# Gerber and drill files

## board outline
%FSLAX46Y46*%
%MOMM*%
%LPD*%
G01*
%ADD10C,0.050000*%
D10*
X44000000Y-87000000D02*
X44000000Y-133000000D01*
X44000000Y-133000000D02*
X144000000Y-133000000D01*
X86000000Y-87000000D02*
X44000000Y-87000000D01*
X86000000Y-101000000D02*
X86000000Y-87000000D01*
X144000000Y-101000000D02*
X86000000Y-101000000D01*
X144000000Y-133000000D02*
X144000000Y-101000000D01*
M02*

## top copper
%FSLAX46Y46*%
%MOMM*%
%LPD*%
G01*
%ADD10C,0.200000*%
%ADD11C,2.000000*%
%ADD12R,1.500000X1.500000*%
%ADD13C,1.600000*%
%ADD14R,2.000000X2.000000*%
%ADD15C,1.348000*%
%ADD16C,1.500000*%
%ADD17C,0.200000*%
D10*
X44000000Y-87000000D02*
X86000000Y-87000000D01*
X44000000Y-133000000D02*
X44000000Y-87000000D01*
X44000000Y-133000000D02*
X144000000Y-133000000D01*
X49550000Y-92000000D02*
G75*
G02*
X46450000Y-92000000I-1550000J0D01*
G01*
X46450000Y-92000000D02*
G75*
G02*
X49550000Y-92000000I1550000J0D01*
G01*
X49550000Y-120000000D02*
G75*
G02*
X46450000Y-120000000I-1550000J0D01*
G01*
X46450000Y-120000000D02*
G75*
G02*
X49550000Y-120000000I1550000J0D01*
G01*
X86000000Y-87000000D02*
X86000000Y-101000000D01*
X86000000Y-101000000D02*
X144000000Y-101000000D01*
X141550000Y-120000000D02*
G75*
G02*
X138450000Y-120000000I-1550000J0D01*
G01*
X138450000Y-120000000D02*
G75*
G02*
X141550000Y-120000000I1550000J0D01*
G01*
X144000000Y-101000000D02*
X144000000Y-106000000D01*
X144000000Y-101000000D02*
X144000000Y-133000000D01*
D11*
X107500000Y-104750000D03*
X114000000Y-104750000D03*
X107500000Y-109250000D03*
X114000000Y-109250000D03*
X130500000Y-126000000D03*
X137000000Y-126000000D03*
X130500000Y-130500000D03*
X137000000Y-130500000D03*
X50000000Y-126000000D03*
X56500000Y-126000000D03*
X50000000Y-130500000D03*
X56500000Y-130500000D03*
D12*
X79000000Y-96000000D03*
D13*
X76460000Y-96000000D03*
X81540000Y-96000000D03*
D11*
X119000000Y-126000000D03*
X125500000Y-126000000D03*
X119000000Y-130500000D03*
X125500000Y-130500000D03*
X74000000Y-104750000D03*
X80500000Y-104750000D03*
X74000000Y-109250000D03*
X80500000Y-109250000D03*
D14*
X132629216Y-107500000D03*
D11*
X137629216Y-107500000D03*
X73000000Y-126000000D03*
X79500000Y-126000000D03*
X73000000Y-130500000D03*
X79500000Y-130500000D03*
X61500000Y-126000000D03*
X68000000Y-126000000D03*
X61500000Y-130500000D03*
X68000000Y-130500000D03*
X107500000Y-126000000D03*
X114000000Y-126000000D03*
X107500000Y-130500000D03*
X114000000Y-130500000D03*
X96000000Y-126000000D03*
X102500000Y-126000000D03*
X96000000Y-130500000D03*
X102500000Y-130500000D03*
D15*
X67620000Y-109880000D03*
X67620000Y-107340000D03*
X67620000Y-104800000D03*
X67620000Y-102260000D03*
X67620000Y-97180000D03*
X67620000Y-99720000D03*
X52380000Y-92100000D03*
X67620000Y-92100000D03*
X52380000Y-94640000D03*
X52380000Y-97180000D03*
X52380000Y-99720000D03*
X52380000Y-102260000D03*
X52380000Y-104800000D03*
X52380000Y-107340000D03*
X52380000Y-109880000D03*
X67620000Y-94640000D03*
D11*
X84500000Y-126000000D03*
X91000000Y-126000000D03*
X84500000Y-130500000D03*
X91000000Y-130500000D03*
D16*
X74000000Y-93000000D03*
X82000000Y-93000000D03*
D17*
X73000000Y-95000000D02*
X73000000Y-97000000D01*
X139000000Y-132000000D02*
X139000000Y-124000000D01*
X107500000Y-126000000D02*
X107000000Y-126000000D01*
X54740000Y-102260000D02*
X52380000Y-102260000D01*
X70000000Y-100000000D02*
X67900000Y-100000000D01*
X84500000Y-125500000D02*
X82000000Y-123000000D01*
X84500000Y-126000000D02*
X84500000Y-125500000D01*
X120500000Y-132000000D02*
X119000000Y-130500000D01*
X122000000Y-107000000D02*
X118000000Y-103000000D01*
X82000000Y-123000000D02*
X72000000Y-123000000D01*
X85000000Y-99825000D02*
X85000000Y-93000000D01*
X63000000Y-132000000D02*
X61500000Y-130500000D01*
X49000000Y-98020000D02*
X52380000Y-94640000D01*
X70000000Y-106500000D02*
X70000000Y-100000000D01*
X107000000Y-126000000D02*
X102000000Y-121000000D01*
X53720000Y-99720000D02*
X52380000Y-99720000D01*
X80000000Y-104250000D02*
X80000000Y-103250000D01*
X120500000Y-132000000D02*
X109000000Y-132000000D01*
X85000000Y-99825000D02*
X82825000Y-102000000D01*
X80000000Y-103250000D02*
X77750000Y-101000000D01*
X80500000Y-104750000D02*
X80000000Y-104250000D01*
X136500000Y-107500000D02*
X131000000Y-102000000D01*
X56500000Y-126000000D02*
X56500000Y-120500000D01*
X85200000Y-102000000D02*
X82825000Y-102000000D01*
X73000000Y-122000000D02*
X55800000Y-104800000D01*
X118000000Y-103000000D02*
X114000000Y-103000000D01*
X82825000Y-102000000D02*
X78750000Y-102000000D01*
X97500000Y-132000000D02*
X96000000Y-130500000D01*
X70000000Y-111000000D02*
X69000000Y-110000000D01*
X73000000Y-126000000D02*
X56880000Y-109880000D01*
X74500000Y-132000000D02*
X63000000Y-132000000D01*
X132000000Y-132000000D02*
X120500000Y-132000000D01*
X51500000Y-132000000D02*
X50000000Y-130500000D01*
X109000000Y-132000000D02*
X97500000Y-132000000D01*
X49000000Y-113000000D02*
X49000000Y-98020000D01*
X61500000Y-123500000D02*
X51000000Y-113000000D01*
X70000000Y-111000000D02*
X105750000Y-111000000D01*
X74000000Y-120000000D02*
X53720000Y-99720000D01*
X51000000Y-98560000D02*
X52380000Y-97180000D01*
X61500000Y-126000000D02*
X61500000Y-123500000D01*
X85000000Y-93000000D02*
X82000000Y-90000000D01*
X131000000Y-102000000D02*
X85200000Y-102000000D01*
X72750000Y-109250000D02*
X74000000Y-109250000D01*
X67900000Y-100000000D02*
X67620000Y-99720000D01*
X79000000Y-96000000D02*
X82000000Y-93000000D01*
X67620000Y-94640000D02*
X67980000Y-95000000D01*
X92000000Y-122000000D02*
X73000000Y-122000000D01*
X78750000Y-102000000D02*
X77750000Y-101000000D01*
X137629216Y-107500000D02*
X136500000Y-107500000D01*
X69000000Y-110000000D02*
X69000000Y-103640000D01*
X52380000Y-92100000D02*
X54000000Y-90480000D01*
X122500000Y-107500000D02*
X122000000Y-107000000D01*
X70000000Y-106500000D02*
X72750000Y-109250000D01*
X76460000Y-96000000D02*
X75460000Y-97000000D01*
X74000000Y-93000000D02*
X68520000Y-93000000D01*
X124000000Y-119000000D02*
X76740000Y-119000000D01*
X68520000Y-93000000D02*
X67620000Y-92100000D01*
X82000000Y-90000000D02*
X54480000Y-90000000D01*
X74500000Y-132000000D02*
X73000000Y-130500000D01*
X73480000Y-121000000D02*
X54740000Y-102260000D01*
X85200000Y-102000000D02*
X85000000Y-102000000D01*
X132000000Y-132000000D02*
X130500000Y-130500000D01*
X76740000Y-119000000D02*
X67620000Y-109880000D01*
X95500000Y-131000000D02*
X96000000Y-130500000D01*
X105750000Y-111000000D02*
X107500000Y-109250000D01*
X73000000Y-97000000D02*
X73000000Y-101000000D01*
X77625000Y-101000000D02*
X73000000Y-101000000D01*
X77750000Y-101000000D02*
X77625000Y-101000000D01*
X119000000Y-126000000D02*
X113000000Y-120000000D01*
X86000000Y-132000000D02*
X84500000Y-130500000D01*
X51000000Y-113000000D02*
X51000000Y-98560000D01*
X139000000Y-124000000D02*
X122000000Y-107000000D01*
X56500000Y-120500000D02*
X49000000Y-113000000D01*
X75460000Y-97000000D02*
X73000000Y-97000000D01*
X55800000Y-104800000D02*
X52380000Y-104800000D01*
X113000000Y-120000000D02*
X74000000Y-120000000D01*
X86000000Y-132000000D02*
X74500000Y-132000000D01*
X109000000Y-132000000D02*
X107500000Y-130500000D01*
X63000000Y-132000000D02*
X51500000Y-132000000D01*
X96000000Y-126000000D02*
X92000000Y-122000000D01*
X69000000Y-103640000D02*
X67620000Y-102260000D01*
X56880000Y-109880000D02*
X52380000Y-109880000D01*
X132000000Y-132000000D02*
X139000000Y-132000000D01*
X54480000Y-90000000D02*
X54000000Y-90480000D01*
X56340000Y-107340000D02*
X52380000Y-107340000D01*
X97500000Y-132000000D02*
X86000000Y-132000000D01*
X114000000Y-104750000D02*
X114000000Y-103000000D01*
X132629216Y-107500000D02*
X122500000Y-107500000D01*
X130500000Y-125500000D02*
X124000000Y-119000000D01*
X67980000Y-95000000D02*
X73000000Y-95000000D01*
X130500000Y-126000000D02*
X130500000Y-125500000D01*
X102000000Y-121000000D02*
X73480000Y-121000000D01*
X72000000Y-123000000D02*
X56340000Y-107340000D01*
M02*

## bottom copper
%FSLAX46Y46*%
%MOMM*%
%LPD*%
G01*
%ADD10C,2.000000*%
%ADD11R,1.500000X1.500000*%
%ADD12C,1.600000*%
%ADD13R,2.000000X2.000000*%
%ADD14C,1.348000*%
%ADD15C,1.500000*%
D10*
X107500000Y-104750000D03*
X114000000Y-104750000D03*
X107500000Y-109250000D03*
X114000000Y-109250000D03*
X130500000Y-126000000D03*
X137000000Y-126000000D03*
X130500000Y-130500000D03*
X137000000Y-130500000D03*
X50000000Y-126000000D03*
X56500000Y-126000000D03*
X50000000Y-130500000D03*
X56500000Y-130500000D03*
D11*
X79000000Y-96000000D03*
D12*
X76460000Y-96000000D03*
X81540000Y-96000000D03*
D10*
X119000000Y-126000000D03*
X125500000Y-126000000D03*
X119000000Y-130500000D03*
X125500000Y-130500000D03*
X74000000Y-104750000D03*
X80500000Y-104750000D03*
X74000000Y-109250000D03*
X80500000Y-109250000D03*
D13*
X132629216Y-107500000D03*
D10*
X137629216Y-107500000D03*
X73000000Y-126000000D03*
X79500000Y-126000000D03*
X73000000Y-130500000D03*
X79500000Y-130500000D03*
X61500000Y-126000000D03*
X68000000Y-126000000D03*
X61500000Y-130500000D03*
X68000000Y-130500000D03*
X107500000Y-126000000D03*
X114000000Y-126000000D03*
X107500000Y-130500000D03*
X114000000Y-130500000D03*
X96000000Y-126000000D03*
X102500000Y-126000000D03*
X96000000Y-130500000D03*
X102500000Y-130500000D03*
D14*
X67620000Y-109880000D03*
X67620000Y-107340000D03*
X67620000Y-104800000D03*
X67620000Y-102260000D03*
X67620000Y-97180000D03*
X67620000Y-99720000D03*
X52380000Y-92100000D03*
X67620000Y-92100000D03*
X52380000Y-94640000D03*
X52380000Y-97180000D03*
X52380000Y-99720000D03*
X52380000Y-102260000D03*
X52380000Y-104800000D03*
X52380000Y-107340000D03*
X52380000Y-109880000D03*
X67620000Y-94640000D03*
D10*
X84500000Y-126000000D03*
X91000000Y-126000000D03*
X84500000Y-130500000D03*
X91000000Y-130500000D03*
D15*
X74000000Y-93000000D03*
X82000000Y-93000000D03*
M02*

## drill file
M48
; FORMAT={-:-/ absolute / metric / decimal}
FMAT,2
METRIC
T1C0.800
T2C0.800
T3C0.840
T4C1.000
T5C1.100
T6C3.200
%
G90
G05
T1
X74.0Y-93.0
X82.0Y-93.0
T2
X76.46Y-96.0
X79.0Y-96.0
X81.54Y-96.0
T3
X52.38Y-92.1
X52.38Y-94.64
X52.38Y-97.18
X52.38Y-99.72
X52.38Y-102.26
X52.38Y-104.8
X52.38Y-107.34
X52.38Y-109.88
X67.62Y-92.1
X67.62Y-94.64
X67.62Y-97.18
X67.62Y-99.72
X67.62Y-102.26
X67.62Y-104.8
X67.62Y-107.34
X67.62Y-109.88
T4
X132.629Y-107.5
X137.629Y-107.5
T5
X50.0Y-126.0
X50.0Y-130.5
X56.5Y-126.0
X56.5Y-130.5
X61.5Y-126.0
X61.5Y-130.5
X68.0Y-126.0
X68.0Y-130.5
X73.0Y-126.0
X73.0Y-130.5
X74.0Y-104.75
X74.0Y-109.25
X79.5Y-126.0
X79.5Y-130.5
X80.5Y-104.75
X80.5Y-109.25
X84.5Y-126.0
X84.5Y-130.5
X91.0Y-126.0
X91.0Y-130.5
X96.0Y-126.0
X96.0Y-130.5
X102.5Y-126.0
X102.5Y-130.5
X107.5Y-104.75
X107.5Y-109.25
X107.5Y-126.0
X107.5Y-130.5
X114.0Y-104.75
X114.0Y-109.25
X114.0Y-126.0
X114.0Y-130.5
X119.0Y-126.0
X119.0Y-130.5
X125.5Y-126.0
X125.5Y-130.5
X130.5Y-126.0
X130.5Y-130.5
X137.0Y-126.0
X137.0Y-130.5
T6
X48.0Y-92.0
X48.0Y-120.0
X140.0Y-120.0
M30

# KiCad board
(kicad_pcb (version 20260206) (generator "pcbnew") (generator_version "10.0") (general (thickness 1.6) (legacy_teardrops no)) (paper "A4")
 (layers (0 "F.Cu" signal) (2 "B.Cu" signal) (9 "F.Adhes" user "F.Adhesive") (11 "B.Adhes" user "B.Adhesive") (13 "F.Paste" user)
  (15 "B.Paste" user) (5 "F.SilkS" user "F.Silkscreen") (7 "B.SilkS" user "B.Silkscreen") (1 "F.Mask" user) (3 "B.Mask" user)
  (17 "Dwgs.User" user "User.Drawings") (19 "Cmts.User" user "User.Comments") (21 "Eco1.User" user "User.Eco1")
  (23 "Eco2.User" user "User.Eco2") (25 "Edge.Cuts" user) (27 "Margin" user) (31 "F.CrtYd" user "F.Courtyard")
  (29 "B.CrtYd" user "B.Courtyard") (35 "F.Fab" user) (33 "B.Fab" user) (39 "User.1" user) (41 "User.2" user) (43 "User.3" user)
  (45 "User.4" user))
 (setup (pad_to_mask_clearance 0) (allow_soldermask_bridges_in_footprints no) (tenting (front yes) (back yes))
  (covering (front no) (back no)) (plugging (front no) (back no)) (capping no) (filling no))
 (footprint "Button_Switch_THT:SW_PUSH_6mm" (layer "F.Cu") (at 107.5 104.75)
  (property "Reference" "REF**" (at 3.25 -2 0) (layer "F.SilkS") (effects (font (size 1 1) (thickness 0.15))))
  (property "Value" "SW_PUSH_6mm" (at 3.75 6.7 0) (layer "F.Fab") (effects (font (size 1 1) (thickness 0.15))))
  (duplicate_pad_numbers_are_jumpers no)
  (pad "1" thru_hole circle (at 0 0 90) (size 2 2) (drill 1.1) (layers "*.Cu" "*.Mask") (remove_unused_layers no))
  (pad "1" thru_hole circle (at 6.5 0 90) (size 2 2) (drill 1.1) (layers "*.Cu" "*.Mask") (remove_unused_layers no))
  (pad "2" thru_hole circle (at 0 4.5 90) (size 2 2) (drill 1.1) (layers "*.Cu" "*.Mask") (remove_unused_layers no))
  (pad "2" thru_hole circle (at 6.5 4.5 90) (size 2 2) (drill 1.1) (layers "*.Cu" "*.Mask") (remove_unused_layers no)))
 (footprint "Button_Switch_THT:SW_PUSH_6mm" (layer "F.Cu") (at 130.5 126)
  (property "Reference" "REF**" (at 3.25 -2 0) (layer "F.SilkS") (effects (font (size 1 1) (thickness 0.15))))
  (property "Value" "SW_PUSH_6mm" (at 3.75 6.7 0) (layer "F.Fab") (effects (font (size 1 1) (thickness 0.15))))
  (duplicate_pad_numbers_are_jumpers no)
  (pad "1" thru_hole circle (at 0 0 90) (size 2 2) (drill 1.1) (layers "*.Cu" "*.Mask") (remove_unused_layers no))
  (pad "1" thru_hole circle (at 6.5 0 90) (size 2 2) (drill 1.1) (layers "*.Cu" "*.Mask") (remove_unused_layers no))
  (pad "2" thru_hole circle (at 0 4.5 90) (size 2 2) (drill 1.1) (layers "*.Cu" "*.Mask") (remove_unused_layers no))
  (pad "2" thru_hole circle (at 6.5 4.5 90) (size 2 2) (drill 1.1) (layers "*.Cu" "*.Mask") (remove_unused_layers no)))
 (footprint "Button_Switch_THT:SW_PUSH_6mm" (layer "F.Cu") (at 50 126)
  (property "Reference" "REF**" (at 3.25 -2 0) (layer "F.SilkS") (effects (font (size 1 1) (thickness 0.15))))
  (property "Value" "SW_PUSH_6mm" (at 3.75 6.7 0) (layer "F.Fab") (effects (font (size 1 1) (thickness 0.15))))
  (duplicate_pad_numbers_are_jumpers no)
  (pad "1" thru_hole circle (at 0 0 90) (size 2 2) (drill 1.1) (layers "*.Cu" "*.Mask") (remove_unused_layers no))
  (pad "1" thru_hole circle (at 6.5 0 90) (size 2 2) (drill 1.1) (layers "*.Cu" "*.Mask") (remove_unused_layers no))
  (pad "2" thru_hole circle (at 0 4.5 90) (size 2 2) (drill 1.1) (layers "*.Cu" "*.Mask") (remove_unused_layers no))
  (pad "2" thru_hole circle (at 6.5 4.5 90) (size 2 2) (drill 1.1) (layers "*.Cu" "*.Mask") (remove_unused_layers no)))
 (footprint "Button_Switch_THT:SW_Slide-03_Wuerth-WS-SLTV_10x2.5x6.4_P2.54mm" (layer "F.Cu") (at 79 96)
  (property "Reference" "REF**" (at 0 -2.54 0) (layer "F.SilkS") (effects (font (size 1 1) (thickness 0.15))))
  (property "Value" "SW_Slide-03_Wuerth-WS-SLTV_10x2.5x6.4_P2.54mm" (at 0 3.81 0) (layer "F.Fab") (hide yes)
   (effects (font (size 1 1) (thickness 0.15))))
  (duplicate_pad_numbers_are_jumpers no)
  (pad "1" thru_hole rect (at 0 0) (size 1.5 1.5) (drill 0.8) (layers "*.Cu" "*.Mask") (remove_unused_layers no))
  (pad "2" thru_hole circle (at -2.54 0) (size 1.6 1.6) (drill 0.8) (layers "*.Cu" "*.Mask") (remove_unused_layers no))
  (pad "3" thru_hole circle (at 2.54 0) (size 1.6 1.6) (drill 0.8) (layers "*.Cu" "*.Mask") (remove_unused_layers no)))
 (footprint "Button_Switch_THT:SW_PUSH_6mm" (layer "F.Cu") (at 119 126)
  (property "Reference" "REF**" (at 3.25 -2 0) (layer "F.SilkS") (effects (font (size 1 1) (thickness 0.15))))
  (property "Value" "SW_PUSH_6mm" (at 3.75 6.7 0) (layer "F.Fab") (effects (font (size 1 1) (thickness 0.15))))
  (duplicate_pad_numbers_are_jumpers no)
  (pad "1" thru_hole circle (at 0 0 90) (size 2 2) (drill 1.1) (layers "*.Cu" "*.Mask") (remove_unused_layers no))
  (pad "1" thru_hole circle (at 6.5 0 90) (size 2 2) (drill 1.1) (layers "*.Cu" "*.Mask") (remove_unused_layers no))
  (pad "2" thru_hole circle (at 0 4.5 90) (size 2 2) (drill 1.1) (layers "*.Cu" "*.Mask") (remove_unused_layers no))
  (pad "2" thru_hole circle (at 6.5 4.5 90) (size 2 2) (drill 1.1) (layers "*.Cu" "*.Mask") (remove_unused_layers no)))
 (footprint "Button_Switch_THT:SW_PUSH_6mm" (layer "F.Cu") (at 74 104.75)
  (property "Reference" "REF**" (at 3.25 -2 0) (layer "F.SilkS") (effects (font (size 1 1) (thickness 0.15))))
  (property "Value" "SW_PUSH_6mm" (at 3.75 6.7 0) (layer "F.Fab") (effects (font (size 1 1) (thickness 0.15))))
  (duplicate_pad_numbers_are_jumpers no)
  (pad "1" thru_hole circle (at 0 0 90) (size 2 2) (drill 1.1) (layers "*.Cu" "*.Mask") (remove_unused_layers no))
  (pad "1" thru_hole circle (at 6.5 0 90) (size 2 2) (drill 1.1) (layers "*.Cu" "*.Mask") (remove_unused_layers no))
  (pad "2" thru_hole circle (at 0 4.5 90) (size 2 2) (drill 1.1) (layers "*.Cu" "*.Mask") (remove_unused_layers no))
  (pad "2" thru_hole circle (at 6.5 4.5 90) (size 2 2) (drill 1.1) (layers "*.Cu" "*.Mask") (remove_unused_layers no)))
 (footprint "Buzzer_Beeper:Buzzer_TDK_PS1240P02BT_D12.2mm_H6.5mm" (layer "F.Cu") (at 132.629216 107.5)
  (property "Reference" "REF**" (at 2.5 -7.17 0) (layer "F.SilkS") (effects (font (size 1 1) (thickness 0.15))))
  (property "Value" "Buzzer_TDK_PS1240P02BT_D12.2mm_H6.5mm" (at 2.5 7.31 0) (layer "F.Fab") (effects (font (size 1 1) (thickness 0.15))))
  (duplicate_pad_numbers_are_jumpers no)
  (pad "1" thru_hole rect (at 0 0) (size 2 2) (drill 1) (layers "*.Cu" "*.Mask") (remove_unused_layers no))
  (pad "2" thru_hole circle (at 5 0) (size 2 2) (drill 1) (layers "*.Cu" "*.Mask") (remove_unused_layers no)))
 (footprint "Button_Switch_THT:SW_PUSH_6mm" (layer "F.Cu") (at 73 126)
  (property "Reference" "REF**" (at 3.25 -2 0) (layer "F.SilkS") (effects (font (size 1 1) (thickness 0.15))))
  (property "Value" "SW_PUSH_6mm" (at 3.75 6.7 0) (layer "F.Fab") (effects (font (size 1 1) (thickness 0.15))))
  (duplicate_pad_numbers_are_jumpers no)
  (pad "1" thru_hole circle (at 0 0 90) (size 2 2) (drill 1.1) (layers "*.Cu" "*.Mask") (remove_unused_layers no))
  (pad "1" thru_hole circle (at 6.5 0 90) (size 2 2) (drill 1.1) (layers "*.Cu" "*.Mask") (remove_unused_layers no))
  (pad "2" thru_hole circle (at 0 4.5 90) (size 2 2) (drill 1.1) (layers "*.Cu" "*.Mask") (remove_unused_layers no))
  (pad "2" thru_hole circle (at 6.5 4.5 90) (size 2 2) (drill 1.1) (layers "*.Cu" "*.Mask") (remove_unused_layers no)))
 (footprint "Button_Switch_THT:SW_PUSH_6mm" (layer "F.Cu") (at 61.5 126)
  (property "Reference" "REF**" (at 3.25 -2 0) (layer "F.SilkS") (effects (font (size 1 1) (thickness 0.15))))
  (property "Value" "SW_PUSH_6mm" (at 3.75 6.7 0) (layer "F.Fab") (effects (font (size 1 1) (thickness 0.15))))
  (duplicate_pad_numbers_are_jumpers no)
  (pad "1" thru_hole circle (at 0 0 90) (size 2 2) (drill 1.1) (layers "*.Cu" "*.Mask") (remove_unused_layers no))
  (pad "1" thru_hole circle (at 6.5 0 90) (size 2 2) (drill 1.1) (layers "*.Cu" "*.Mask") (remove_unused_layers no))
  (pad "2" thru_hole circle (at 0 4.5 90) (size 2 2) (drill 1.1) (layers "*.Cu" "*.Mask") (remove_unused_layers no))
  (pad "2" thru_hole circle (at 6.5 4.5 90) (size 2 2) (drill 1.1) (layers "*.Cu" "*.Mask") (remove_unused_layers no)))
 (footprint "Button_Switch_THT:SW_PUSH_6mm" (layer "F.Cu") (at 107.5 126)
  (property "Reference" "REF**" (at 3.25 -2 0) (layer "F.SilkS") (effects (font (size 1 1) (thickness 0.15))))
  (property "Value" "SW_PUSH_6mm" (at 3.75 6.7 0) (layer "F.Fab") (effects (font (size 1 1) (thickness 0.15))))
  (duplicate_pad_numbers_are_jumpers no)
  (pad "1" thru_hole circle (at 0 0 90) (size 2 2) (drill 1.1) (layers "*.Cu" "*.Mask") (remove_unused_layers no))
  (pad "1" thru_hole circle (at 6.5 0 90) (size 2 2) (drill 1.1) (layers "*.Cu" "*.Mask") (remove_unused_layers no))
  (pad "2" thru_hole circle (at 0 4.5 90) (size 2 2) (drill 1.1) (layers "*.Cu" "*.Mask") (remove_unused_layers no))
  (pad "2" thru_hole circle (at 6.5 4.5 90) (size 2 2) (drill 1.1) (layers "*.Cu" "*.Mask") (remove_unused_layers no)))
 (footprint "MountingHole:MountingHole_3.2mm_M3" (layer "F.Cu") (at 140 120)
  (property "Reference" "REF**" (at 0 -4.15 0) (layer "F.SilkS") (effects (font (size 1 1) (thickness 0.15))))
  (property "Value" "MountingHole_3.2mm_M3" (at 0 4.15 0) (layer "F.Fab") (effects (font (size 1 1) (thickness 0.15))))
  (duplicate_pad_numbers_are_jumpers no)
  (pad "" np_thru_hole circle (at 0 0) (size 3.2 3.2) (drill 3.2) (layers "*.Cu" "*.Mask")))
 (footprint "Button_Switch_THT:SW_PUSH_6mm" (layer "F.Cu") (at 96 126)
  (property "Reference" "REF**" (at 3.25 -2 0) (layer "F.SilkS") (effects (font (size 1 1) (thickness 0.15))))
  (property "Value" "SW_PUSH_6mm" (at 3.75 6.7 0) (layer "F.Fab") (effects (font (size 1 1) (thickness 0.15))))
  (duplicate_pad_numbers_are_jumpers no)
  (pad "1" thru_hole circle (at 0 0 90) (size 2 2) (drill 1.1) (layers "*.Cu" "*.Mask") (remove_unused_layers no))
  (pad "1" thru_hole circle (at 6.5 0 90) (size 2 2) (drill 1.1) (layers "*.Cu" "*.Mask") (remove_unused_layers no))
  (pad "2" thru_hole circle (at 0 4.5 90) (size 2 2) (drill 1.1) (layers "*.Cu" "*.Mask") (remove_unused_layers no))
  (pad "2" thru_hole circle (at 6.5 4.5 90) (size 2 2) (drill 1.1) (layers "*.Cu" "*.Mask") (remove_unused_layers no)))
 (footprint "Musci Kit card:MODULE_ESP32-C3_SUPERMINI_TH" (layer "F.Cu") (at 60 102)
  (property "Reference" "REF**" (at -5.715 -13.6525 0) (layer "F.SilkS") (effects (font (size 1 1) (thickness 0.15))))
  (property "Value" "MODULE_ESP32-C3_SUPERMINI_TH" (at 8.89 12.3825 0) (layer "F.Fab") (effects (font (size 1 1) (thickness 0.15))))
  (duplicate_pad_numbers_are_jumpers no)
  (pad "0" thru_hole circle (at 7.62 7.88) (size 1.348 1.348) (drill 0.84) (layers "*.Cu" "*.Mask") (remove_unused_layers no)
   (solder_mask_margin 0.102))
  (pad "1" thru_hole circle (at 7.62 5.34) (size 1.348 1.348) (drill 0.84) (layers "*.Cu" "*.Mask") (remove_unused_layers no)
   (solder_mask_margin 0.102))
  (pad "2" thru_hole circle (at 7.62 2.8) (size 1.348 1.348) (drill 0.84) (layers "*.Cu" "*.Mask") (remove_unused_layers no)
   (solder_mask_margin 0.102))
  (pad "3" thru_hole circle (at 7.62 0.26) (size 1.348 1.348) (drill 0.84) (layers "*.Cu" "*.Mask") (remove_unused_layers no)
   (solder_mask_margin 0.102))
  (pad "3.3" thru_hole circle (at 7.62 -4.82) (size 1.348 1.348) (drill 0.84) (layers "*.Cu" "*.Mask") (remove_unused_layers no)
   (solder_mask_margin 0.102))
  (pad "4" thru_hole circle (at 7.62 -2.28) (size 1.348 1.348) (drill 0.84) (layers "*.Cu" "*.Mask") (remove_unused_layers no)
   (solder_mask_margin 0.102))
  (pad "5" thru_hole circle (at -7.62 -9.9) (size 1.348 1.348) (drill 0.84) (layers "*.Cu" "*.Mask") (remove_unused_layers no)
   (solder_mask_margin 0.102))
  (pad "5V" thru_hole circle (at 7.62 -9.9) (size 1.348 1.348) (drill 0.84) (layers "*.Cu" "*.Mask") (remove_unused_layers no)
   (solder_mask_margin 0.102))
  (pad "6" thru_hole circle (at -7.62 -7.36) (size 1.348 1.348) (drill 0.84) (layers "*.Cu" "*.Mask") (remove_unused_layers no)
   (solder_mask_margin 0.102))
  (pad "7" thru_hole circle (at -7.62 -4.82) (size 1.348 1.348) (drill 0.84) (layers "*.Cu" "*.Mask") (remove_unused_layers no)
   (solder_mask_margin 0.102))
  (pad "8" thru_hole circle (at -7.62 -2.28) (size 1.348 1.348) (drill 0.84) (layers "*.Cu" "*.Mask") (remove_unused_layers no)
   (solder_mask_margin 0.102))
  (pad "9" thru_hole circle (at -7.62 0.26) (size 1.348 1.348) (drill 0.84) (layers "*.Cu" "*.Mask") (remove_unused_layers no)
   (solder_mask_margin 0.102))
  (pad "10" thru_hole circle (at -7.62 2.8) (size 1.348 1.348) (drill 0.84) (layers "*.Cu" "*.Mask") (remove_unused_layers no)
   (solder_mask_margin 0.102))
  (pad "20" thru_hole circle (at -7.62 5.34) (size 1.348 1.348) (drill 0.84) (layers "*.Cu" "*.Mask") (remove_unused_layers no)
   (solder_mask_margin 0.102))
  (pad "21" thru_hole circle (at -7.62 7.88) (size 1.348 1.348) (drill 0.84) (layers "*.Cu" "*.Mask") (remove_unused_layers no)
   (solder_mask_margin 0.102))
  (pad "G" thru_hole circle (at 7.62 -7.36) (size 1.348 1.348) (drill 0.84) (layers "*.Cu" "*.Mask") (remove_unused_layers no)
   (solder_mask_margin 0.102)))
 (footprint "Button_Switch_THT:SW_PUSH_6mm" (layer "F.Cu") (at 84.5 126)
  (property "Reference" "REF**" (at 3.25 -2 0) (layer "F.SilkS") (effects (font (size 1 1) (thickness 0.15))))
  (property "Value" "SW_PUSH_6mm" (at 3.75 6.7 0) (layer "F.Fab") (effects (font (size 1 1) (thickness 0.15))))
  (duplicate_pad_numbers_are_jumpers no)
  (pad "1" thru_hole circle (at 0 0 90) (size 2 2) (drill 1.1) (layers "*.Cu" "*.Mask") (remove_unused_layers no))
  (pad "1" thru_hole circle (at 6.5 0 90) (size 2 2) (drill 1.1) (layers "*.Cu" "*.Mask") (remove_unused_layers no))
  (pad "2" thru_hole circle (at 0 4.5 90) (size 2 2) (drill 1.1) (layers "*.Cu" "*.Mask") (remove_unused_layers no))
  (pad "2" thru_hole circle (at 6.5 4.5 90) (size 2 2) (drill 1.1) (layers "*.Cu" "*.Mask") (remove_unused_layers no)))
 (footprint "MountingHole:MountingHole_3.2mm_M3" (layer "F.Cu") (at 48 92)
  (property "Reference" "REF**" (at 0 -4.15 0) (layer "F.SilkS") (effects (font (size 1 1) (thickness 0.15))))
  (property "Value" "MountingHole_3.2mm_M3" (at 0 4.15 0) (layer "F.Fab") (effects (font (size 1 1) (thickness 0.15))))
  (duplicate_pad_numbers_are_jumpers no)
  (pad "" np_thru_hole circle (at 0 0) (size 3.2 3.2) (drill 3.2) (layers "*.Cu" "*.Mask")))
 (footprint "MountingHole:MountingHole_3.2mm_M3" (layer "F.Cu") (at 48 120)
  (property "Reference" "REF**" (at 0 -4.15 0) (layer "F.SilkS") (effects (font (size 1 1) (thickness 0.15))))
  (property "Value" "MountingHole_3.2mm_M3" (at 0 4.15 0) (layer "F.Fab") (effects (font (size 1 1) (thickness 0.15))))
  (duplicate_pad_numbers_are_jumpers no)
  (pad "" np_thru_hole circle (at 0 0) (size 3.2 3.2) (drill 3.2) (layers "*.Cu" "*.Mask")))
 (gr_line (start 44 87) (end 86 87) (stroke (width 0.2) (type default)) (layer "F.Cu"))
 (gr_line (start 44 133) (end 44 87) (stroke (width 0.2) (type default)) (layer "F.Cu"))
 (gr_line (start 44 133) (end 144 133) (stroke (width 0.2) (type default)) (layer "F.Cu"))
 (gr_circle (center 48 92) (end 49.55 92) (stroke (width 0.2) (type solid)) (fill no) (layer "F.Cu"))
 (gr_circle (center 48 120) (end 49.55 120) (stroke (width 0.2) (type solid)) (fill no) (layer "F.Cu"))
 (gr_line (start 86 87) (end 86 101) (stroke (width 0.2) (type default)) (layer "F.Cu"))
 (gr_line (start 86 101) (end 144 101) (stroke (width 0.2) (type default)) (layer "F.Cu"))
 (gr_circle (center 140 120) (end 141.55 120) (stroke (width 0.2) (type solid)) (fill no) (layer "F.Cu"))
 (gr_line (start 144 101) (end 144 106) (stroke (width 0.2) (type default)) (layer "F.Cu"))
 (gr_line (start 144 101) (end 144 133) (stroke (width 0.2) (type default)) (layer "F.Cu"))
 (gr_line (start 44 87) (end 44 133) (stroke (width 0.05) (type default)) (layer "Edge.Cuts"))
 (gr_line (start 44 133) (end 144 133) (stroke (width 0.05) (type default)) (layer "Edge.Cuts"))
 (gr_line (start 86 87) (end 44 87) (stroke (width 0.05) (type default)) (layer "Edge.Cuts"))
 (gr_line (start 86 101) (end 86 87) (stroke (width 0.05) (type default)) (layer "Edge.Cuts"))
 (gr_line (start 144 101) (end 86 101) (stroke (width 0.05) (type default)) (layer "Edge.Cuts"))
 (gr_line (start 144 133) (end 144 101) (stroke (width 0.05) (type default)) (layer "Edge.Cuts"))
 (segment (start 73 95) (end 73 97) (width 0.2) (layer "F.Cu") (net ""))
 (segment (start 139 132) (end 139 124) (width 0.2) (layer "F.Cu") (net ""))
 (segment (start 107.5 126) (end 107 126) (width 0.2) (layer "F.Cu") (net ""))
 (segment (start 54.74 102.26) (end 52.38 102.26) (width 0.2) (layer "F.Cu") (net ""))
 (segment (start 70 100) (end 67.9 100) (width 0.2) (layer "F.Cu") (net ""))
 (segment (start 84.5 125.5) (end 82 123) (width 0.2) (layer "F.Cu") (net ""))
 (segment (start 84.5 126) (end 84.5 125.5) (width 0.2) (layer "F.Cu") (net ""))
 (segment (start 120.5 132) (end 119 130.5) (width 0.2) (layer "F.Cu") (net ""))
 (segment (start 122 107) (end 118 103) (width 0.2) (layer "F.Cu") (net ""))
 (segment (start 82 123) (end 72 123) (width 0.2) (layer "F.Cu") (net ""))
 (segment (start 85 99.825) (end 85 93) (width 0.2) (layer "F.Cu") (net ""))
 (segment (start 63 132) (end 61.5 130.5) (width 0.2) (layer "F.Cu") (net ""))
 (segment (start 49 98.02) (end 52.38 94.64) (width 0.2) (layer "F.Cu") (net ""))
 (segment (start 70 106.5) (end 70 100) (width 0.2) (layer "F.Cu") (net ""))
 (segment (start 107 126) (end 102 121) (width 0.2) (layer "F.Cu") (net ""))
 (segment (start 53.72 99.72) (end 52.38 99.72) (width 0.2) (layer "F.Cu") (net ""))
 (segment (start 80 104.25) (end 80 103.25) (width 0.2) (layer "F.Cu") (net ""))
 (segment (start 120.5 132) (end 109 132) (width 0.2) (layer "F.Cu") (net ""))
 (segment (start 85 99.825) (end 82.825 102) (width 0.2) (layer "F.Cu") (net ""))
 (segment (start 80 103.25) (end 77.75 101) (width 0.2) (layer "F.Cu") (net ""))
 (segment (start 80.5 104.75) (end 80 104.25) (width 0.2) (layer "F.Cu") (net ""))
 (segment (start 136.5 107.5) (end 131 102) (width 0.2) (layer "F.Cu") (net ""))
 (segment (start 56.5 126) (end 56.5 120.5) (width 0.2) (layer "F.Cu") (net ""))
 (segment (start 85.2 102) (end 82.825 102) (width 0.2) (layer "F.Cu") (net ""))
 (segment (start 73 122) (end 55.8 104.8) (width 0.2) (layer "F.Cu") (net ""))
 (segment (start 118 103) (end 114 103) (width 0.2) (layer "F.Cu") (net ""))
 (segment (start 82.825 102) (end 78.75 102) (width 0.2) (layer "F.Cu") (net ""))
 (segment (start 97.5 132) (end 96 130.5) (width 0.2) (layer "F.Cu") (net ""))
 (segment (start 70 111) (end 69 110) (width 0.2) (layer "F.Cu") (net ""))
 (segment (start 73 126) (end 56.88 109.88) (width 0.2) (layer "F.Cu") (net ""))
 (segment (start 74.5 132) (end 63 132) (width 0.2) (layer "F.Cu") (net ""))
 (segment (start 132 132) (end 120.5 132) (width 0.2) (layer "F.Cu") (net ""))
 (segment (start 51.5 132) (end 50 130.5) (width 0.2) (layer "F.Cu") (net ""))
 (segment (start 109 132) (end 97.5 132) (width 0.2) (layer "F.Cu") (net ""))
 (segment (start 49 113) (end 49 98.02) (width 0.2) (layer "F.Cu") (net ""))
 (segment (start 61.5 123.5) (end 51 113) (width 0.2) (layer "F.Cu") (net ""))
 (segment (start 70 111) (end 105.75 111) (width 0.2) (layer "F.Cu") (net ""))
 (segment (start 74 120) (end 53.72 99.72) (width 0.2) (layer "F.Cu") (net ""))
 (segment (start 51 98.56) (end 52.38 97.18) (width 0.2) (layer "F.Cu") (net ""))
 (segment (start 61.5 126) (end 61.5 123.5) (width 0.2) (layer "F.Cu") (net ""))
 (segment (start 85 93) (end 82 90) (width 0.2) (layer "F.Cu") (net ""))
 (segment (start 131 102) (end 85.2 102) (width 0.2) (layer "F.Cu") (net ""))
 (segment (start 72.75 109.25) (end 74 109.25) (width 0.2) (layer "F.Cu") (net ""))
 (segment (start 67.9 100) (end 67.62 99.72) (width 0.2) (layer "F.Cu") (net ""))
 (segment (start 79 96) (end 82 93) (width 0.2) (layer "F.Cu") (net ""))
 (segment (start 67.62 94.64) (end 67.98 95) (width 0.2) (layer "F.Cu") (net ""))
 (segment (start 92 122) (end 73 122) (width 0.2) (layer "F.Cu") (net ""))
 (segment (start 78.75 102) (end 77.75 101) (width 0.2) (layer "F.Cu") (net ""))
 (segment (start 137.629216 107.5) (end 136.5 107.5) (width 0.2) (layer "F.Cu") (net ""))
 (segment (start 69 110) (end 69 103.64) (width 0.2) (layer "F.Cu") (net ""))
 (segment (start 52.38 92.1) (end 54 90.48) (width 0.2) (layer "F.Cu") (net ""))
 (segment (start 122.5 107.5) (end 122 107) (width 0.2) (layer "F.Cu") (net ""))
 (segment (start 70 106.5) (end 72.75 109.25) (width 0.2) (layer "F.Cu") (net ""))
 (segment (start 76.46 96) (end 75.46 97) (width 0.2) (layer "F.Cu") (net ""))
 (segment (start 74 93) (end 68.52 93) (width 0.2) (layer "F.Cu") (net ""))
 (segment (start 124 119) (end 76.74 119) (width 0.2) (layer "F.Cu") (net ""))
 (segment (start 68.52 93) (end 67.62 92.1) (width 0.2) (layer "F.Cu") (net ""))
 (segment (start 82 90) (end 54.48 90) (width 0.2) (layer "F.Cu") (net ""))
 (segment (start 74.5 132) (end 73 130.5) (width 0.2) (layer "F.Cu") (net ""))
 (segment (start 73.48 121) (end 54.74 102.26) (width 0.2) (layer "F.Cu") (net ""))
 (segment (start 85.2 102) (end 85 102) (width 0.2) (layer "F.Cu") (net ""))
 (segment (start 132 132) (end 130.5 130.5) (width 0.2) (layer "F.Cu") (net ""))
 (segment (start 76.74 119) (end 67.62 109.88) (width 0.2) (layer "F.Cu") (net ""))
 (segment (start 95.5 131) (end 96 130.5) (width 0.2) (layer "F.Cu") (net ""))
 (segment (start 105.75 111) (end 107.5 109.25) (width 0.2) (layer "F.Cu") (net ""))
 (segment (start 73 97) (end 73 101) (width 0.2) (layer "F.Cu") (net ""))
 (segment (start 77.625 101) (end 73 101) (width 0.2) (layer "F.Cu") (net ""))
 (segment (start 77.75 101) (end 77.625 101) (width 0.2) (layer "F.Cu") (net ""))
 (segment (start 119 126) (end 113 120) (width 0.2) (layer "F.Cu") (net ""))
 (segment (start 86 132) (end 84.5 130.5) (width 0.2) (layer "F.Cu") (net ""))
 (segment (start 51 113) (end 51 98.56) (width 0.2) (layer "F.Cu") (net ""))
 (segment (start 139 124) (end 122 107) (width 0.2) (layer "F.Cu") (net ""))
 (segment (start 56.5 120.5) (end 49 113) (width 0.2) (layer "F.Cu") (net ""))
 (segment (start 75.46 97) (end 73 97) (width 0.2) (layer "F.Cu") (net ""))
 (segment (start 55.8 104.8) (end 52.38 104.8) (width 0.2) (layer "F.Cu") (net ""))
 (segment (start 113 120) (end 74 120) (width 0.2) (layer "F.Cu") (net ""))
 (segment (start 86 132) (end 74.5 132) (width 0.2) (layer "F.Cu") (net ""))
 (segment (start 109 132) (end 107.5 130.5) (width 0.2) (layer "F.Cu") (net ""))
 (segment (start 63 132) (end 51.5 132) (width 0.2) (layer "F.Cu") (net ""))
 (segment (start 96 126) (end 92 122) (width 0.2) (layer "F.Cu") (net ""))
 (segment (start 69 103.64) (end 67.62 102.26) (width 0.2) (layer "F.Cu") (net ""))
 (segment (start 56.88 109.88) (end 52.38 109.88) (width 0.2) (layer "F.Cu") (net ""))
 (segment (start 132 132) (end 139 132) (width 0.2) (layer "F.Cu") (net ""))
 (segment (start 54.48 90) (end 54 90.48) (width 0.2) (layer "F.Cu") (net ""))
 (segment (start 56.34 107.34) (end 52.38 107.34) (width 0.2) (layer "F.Cu") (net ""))
 (segment (start 97.5 132) (end 86 132) (width 0.2) (layer "F.Cu") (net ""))
 (segment (start 114 104.75) (end 114 103) (width 0.2) (layer "F.Cu") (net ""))
 (segment (start 132.629216 107.5) (end 122.5 107.5) (width 0.2) (layer "F.Cu") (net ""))
 (segment (start 130.5 125.5) (end 124 119) (width 0.2) (layer "F.Cu") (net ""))
 (segment (start 67.98 95) (end 73 95) (width 0.2) (layer "F.Cu") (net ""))
 (segment (start 130.5 126) (end 130.5 125.5) (width 0.2) (layer "F.Cu") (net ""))
 (segment (start 102 121) (end 73.48 121) (width 0.2) (layer "F.Cu") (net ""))
 (segment (start 72 123) (end 56.34 107.34) (width 0.2) (layer "F.Cu") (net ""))
 (via (at 74 93) (size 1.5) (drill 0.8) (layers "F.Cu" "B.Cu") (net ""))
 (via (at 82 93) (size 1.5) (drill 0.8) (layers "F.Cu" "B.Cu") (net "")))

